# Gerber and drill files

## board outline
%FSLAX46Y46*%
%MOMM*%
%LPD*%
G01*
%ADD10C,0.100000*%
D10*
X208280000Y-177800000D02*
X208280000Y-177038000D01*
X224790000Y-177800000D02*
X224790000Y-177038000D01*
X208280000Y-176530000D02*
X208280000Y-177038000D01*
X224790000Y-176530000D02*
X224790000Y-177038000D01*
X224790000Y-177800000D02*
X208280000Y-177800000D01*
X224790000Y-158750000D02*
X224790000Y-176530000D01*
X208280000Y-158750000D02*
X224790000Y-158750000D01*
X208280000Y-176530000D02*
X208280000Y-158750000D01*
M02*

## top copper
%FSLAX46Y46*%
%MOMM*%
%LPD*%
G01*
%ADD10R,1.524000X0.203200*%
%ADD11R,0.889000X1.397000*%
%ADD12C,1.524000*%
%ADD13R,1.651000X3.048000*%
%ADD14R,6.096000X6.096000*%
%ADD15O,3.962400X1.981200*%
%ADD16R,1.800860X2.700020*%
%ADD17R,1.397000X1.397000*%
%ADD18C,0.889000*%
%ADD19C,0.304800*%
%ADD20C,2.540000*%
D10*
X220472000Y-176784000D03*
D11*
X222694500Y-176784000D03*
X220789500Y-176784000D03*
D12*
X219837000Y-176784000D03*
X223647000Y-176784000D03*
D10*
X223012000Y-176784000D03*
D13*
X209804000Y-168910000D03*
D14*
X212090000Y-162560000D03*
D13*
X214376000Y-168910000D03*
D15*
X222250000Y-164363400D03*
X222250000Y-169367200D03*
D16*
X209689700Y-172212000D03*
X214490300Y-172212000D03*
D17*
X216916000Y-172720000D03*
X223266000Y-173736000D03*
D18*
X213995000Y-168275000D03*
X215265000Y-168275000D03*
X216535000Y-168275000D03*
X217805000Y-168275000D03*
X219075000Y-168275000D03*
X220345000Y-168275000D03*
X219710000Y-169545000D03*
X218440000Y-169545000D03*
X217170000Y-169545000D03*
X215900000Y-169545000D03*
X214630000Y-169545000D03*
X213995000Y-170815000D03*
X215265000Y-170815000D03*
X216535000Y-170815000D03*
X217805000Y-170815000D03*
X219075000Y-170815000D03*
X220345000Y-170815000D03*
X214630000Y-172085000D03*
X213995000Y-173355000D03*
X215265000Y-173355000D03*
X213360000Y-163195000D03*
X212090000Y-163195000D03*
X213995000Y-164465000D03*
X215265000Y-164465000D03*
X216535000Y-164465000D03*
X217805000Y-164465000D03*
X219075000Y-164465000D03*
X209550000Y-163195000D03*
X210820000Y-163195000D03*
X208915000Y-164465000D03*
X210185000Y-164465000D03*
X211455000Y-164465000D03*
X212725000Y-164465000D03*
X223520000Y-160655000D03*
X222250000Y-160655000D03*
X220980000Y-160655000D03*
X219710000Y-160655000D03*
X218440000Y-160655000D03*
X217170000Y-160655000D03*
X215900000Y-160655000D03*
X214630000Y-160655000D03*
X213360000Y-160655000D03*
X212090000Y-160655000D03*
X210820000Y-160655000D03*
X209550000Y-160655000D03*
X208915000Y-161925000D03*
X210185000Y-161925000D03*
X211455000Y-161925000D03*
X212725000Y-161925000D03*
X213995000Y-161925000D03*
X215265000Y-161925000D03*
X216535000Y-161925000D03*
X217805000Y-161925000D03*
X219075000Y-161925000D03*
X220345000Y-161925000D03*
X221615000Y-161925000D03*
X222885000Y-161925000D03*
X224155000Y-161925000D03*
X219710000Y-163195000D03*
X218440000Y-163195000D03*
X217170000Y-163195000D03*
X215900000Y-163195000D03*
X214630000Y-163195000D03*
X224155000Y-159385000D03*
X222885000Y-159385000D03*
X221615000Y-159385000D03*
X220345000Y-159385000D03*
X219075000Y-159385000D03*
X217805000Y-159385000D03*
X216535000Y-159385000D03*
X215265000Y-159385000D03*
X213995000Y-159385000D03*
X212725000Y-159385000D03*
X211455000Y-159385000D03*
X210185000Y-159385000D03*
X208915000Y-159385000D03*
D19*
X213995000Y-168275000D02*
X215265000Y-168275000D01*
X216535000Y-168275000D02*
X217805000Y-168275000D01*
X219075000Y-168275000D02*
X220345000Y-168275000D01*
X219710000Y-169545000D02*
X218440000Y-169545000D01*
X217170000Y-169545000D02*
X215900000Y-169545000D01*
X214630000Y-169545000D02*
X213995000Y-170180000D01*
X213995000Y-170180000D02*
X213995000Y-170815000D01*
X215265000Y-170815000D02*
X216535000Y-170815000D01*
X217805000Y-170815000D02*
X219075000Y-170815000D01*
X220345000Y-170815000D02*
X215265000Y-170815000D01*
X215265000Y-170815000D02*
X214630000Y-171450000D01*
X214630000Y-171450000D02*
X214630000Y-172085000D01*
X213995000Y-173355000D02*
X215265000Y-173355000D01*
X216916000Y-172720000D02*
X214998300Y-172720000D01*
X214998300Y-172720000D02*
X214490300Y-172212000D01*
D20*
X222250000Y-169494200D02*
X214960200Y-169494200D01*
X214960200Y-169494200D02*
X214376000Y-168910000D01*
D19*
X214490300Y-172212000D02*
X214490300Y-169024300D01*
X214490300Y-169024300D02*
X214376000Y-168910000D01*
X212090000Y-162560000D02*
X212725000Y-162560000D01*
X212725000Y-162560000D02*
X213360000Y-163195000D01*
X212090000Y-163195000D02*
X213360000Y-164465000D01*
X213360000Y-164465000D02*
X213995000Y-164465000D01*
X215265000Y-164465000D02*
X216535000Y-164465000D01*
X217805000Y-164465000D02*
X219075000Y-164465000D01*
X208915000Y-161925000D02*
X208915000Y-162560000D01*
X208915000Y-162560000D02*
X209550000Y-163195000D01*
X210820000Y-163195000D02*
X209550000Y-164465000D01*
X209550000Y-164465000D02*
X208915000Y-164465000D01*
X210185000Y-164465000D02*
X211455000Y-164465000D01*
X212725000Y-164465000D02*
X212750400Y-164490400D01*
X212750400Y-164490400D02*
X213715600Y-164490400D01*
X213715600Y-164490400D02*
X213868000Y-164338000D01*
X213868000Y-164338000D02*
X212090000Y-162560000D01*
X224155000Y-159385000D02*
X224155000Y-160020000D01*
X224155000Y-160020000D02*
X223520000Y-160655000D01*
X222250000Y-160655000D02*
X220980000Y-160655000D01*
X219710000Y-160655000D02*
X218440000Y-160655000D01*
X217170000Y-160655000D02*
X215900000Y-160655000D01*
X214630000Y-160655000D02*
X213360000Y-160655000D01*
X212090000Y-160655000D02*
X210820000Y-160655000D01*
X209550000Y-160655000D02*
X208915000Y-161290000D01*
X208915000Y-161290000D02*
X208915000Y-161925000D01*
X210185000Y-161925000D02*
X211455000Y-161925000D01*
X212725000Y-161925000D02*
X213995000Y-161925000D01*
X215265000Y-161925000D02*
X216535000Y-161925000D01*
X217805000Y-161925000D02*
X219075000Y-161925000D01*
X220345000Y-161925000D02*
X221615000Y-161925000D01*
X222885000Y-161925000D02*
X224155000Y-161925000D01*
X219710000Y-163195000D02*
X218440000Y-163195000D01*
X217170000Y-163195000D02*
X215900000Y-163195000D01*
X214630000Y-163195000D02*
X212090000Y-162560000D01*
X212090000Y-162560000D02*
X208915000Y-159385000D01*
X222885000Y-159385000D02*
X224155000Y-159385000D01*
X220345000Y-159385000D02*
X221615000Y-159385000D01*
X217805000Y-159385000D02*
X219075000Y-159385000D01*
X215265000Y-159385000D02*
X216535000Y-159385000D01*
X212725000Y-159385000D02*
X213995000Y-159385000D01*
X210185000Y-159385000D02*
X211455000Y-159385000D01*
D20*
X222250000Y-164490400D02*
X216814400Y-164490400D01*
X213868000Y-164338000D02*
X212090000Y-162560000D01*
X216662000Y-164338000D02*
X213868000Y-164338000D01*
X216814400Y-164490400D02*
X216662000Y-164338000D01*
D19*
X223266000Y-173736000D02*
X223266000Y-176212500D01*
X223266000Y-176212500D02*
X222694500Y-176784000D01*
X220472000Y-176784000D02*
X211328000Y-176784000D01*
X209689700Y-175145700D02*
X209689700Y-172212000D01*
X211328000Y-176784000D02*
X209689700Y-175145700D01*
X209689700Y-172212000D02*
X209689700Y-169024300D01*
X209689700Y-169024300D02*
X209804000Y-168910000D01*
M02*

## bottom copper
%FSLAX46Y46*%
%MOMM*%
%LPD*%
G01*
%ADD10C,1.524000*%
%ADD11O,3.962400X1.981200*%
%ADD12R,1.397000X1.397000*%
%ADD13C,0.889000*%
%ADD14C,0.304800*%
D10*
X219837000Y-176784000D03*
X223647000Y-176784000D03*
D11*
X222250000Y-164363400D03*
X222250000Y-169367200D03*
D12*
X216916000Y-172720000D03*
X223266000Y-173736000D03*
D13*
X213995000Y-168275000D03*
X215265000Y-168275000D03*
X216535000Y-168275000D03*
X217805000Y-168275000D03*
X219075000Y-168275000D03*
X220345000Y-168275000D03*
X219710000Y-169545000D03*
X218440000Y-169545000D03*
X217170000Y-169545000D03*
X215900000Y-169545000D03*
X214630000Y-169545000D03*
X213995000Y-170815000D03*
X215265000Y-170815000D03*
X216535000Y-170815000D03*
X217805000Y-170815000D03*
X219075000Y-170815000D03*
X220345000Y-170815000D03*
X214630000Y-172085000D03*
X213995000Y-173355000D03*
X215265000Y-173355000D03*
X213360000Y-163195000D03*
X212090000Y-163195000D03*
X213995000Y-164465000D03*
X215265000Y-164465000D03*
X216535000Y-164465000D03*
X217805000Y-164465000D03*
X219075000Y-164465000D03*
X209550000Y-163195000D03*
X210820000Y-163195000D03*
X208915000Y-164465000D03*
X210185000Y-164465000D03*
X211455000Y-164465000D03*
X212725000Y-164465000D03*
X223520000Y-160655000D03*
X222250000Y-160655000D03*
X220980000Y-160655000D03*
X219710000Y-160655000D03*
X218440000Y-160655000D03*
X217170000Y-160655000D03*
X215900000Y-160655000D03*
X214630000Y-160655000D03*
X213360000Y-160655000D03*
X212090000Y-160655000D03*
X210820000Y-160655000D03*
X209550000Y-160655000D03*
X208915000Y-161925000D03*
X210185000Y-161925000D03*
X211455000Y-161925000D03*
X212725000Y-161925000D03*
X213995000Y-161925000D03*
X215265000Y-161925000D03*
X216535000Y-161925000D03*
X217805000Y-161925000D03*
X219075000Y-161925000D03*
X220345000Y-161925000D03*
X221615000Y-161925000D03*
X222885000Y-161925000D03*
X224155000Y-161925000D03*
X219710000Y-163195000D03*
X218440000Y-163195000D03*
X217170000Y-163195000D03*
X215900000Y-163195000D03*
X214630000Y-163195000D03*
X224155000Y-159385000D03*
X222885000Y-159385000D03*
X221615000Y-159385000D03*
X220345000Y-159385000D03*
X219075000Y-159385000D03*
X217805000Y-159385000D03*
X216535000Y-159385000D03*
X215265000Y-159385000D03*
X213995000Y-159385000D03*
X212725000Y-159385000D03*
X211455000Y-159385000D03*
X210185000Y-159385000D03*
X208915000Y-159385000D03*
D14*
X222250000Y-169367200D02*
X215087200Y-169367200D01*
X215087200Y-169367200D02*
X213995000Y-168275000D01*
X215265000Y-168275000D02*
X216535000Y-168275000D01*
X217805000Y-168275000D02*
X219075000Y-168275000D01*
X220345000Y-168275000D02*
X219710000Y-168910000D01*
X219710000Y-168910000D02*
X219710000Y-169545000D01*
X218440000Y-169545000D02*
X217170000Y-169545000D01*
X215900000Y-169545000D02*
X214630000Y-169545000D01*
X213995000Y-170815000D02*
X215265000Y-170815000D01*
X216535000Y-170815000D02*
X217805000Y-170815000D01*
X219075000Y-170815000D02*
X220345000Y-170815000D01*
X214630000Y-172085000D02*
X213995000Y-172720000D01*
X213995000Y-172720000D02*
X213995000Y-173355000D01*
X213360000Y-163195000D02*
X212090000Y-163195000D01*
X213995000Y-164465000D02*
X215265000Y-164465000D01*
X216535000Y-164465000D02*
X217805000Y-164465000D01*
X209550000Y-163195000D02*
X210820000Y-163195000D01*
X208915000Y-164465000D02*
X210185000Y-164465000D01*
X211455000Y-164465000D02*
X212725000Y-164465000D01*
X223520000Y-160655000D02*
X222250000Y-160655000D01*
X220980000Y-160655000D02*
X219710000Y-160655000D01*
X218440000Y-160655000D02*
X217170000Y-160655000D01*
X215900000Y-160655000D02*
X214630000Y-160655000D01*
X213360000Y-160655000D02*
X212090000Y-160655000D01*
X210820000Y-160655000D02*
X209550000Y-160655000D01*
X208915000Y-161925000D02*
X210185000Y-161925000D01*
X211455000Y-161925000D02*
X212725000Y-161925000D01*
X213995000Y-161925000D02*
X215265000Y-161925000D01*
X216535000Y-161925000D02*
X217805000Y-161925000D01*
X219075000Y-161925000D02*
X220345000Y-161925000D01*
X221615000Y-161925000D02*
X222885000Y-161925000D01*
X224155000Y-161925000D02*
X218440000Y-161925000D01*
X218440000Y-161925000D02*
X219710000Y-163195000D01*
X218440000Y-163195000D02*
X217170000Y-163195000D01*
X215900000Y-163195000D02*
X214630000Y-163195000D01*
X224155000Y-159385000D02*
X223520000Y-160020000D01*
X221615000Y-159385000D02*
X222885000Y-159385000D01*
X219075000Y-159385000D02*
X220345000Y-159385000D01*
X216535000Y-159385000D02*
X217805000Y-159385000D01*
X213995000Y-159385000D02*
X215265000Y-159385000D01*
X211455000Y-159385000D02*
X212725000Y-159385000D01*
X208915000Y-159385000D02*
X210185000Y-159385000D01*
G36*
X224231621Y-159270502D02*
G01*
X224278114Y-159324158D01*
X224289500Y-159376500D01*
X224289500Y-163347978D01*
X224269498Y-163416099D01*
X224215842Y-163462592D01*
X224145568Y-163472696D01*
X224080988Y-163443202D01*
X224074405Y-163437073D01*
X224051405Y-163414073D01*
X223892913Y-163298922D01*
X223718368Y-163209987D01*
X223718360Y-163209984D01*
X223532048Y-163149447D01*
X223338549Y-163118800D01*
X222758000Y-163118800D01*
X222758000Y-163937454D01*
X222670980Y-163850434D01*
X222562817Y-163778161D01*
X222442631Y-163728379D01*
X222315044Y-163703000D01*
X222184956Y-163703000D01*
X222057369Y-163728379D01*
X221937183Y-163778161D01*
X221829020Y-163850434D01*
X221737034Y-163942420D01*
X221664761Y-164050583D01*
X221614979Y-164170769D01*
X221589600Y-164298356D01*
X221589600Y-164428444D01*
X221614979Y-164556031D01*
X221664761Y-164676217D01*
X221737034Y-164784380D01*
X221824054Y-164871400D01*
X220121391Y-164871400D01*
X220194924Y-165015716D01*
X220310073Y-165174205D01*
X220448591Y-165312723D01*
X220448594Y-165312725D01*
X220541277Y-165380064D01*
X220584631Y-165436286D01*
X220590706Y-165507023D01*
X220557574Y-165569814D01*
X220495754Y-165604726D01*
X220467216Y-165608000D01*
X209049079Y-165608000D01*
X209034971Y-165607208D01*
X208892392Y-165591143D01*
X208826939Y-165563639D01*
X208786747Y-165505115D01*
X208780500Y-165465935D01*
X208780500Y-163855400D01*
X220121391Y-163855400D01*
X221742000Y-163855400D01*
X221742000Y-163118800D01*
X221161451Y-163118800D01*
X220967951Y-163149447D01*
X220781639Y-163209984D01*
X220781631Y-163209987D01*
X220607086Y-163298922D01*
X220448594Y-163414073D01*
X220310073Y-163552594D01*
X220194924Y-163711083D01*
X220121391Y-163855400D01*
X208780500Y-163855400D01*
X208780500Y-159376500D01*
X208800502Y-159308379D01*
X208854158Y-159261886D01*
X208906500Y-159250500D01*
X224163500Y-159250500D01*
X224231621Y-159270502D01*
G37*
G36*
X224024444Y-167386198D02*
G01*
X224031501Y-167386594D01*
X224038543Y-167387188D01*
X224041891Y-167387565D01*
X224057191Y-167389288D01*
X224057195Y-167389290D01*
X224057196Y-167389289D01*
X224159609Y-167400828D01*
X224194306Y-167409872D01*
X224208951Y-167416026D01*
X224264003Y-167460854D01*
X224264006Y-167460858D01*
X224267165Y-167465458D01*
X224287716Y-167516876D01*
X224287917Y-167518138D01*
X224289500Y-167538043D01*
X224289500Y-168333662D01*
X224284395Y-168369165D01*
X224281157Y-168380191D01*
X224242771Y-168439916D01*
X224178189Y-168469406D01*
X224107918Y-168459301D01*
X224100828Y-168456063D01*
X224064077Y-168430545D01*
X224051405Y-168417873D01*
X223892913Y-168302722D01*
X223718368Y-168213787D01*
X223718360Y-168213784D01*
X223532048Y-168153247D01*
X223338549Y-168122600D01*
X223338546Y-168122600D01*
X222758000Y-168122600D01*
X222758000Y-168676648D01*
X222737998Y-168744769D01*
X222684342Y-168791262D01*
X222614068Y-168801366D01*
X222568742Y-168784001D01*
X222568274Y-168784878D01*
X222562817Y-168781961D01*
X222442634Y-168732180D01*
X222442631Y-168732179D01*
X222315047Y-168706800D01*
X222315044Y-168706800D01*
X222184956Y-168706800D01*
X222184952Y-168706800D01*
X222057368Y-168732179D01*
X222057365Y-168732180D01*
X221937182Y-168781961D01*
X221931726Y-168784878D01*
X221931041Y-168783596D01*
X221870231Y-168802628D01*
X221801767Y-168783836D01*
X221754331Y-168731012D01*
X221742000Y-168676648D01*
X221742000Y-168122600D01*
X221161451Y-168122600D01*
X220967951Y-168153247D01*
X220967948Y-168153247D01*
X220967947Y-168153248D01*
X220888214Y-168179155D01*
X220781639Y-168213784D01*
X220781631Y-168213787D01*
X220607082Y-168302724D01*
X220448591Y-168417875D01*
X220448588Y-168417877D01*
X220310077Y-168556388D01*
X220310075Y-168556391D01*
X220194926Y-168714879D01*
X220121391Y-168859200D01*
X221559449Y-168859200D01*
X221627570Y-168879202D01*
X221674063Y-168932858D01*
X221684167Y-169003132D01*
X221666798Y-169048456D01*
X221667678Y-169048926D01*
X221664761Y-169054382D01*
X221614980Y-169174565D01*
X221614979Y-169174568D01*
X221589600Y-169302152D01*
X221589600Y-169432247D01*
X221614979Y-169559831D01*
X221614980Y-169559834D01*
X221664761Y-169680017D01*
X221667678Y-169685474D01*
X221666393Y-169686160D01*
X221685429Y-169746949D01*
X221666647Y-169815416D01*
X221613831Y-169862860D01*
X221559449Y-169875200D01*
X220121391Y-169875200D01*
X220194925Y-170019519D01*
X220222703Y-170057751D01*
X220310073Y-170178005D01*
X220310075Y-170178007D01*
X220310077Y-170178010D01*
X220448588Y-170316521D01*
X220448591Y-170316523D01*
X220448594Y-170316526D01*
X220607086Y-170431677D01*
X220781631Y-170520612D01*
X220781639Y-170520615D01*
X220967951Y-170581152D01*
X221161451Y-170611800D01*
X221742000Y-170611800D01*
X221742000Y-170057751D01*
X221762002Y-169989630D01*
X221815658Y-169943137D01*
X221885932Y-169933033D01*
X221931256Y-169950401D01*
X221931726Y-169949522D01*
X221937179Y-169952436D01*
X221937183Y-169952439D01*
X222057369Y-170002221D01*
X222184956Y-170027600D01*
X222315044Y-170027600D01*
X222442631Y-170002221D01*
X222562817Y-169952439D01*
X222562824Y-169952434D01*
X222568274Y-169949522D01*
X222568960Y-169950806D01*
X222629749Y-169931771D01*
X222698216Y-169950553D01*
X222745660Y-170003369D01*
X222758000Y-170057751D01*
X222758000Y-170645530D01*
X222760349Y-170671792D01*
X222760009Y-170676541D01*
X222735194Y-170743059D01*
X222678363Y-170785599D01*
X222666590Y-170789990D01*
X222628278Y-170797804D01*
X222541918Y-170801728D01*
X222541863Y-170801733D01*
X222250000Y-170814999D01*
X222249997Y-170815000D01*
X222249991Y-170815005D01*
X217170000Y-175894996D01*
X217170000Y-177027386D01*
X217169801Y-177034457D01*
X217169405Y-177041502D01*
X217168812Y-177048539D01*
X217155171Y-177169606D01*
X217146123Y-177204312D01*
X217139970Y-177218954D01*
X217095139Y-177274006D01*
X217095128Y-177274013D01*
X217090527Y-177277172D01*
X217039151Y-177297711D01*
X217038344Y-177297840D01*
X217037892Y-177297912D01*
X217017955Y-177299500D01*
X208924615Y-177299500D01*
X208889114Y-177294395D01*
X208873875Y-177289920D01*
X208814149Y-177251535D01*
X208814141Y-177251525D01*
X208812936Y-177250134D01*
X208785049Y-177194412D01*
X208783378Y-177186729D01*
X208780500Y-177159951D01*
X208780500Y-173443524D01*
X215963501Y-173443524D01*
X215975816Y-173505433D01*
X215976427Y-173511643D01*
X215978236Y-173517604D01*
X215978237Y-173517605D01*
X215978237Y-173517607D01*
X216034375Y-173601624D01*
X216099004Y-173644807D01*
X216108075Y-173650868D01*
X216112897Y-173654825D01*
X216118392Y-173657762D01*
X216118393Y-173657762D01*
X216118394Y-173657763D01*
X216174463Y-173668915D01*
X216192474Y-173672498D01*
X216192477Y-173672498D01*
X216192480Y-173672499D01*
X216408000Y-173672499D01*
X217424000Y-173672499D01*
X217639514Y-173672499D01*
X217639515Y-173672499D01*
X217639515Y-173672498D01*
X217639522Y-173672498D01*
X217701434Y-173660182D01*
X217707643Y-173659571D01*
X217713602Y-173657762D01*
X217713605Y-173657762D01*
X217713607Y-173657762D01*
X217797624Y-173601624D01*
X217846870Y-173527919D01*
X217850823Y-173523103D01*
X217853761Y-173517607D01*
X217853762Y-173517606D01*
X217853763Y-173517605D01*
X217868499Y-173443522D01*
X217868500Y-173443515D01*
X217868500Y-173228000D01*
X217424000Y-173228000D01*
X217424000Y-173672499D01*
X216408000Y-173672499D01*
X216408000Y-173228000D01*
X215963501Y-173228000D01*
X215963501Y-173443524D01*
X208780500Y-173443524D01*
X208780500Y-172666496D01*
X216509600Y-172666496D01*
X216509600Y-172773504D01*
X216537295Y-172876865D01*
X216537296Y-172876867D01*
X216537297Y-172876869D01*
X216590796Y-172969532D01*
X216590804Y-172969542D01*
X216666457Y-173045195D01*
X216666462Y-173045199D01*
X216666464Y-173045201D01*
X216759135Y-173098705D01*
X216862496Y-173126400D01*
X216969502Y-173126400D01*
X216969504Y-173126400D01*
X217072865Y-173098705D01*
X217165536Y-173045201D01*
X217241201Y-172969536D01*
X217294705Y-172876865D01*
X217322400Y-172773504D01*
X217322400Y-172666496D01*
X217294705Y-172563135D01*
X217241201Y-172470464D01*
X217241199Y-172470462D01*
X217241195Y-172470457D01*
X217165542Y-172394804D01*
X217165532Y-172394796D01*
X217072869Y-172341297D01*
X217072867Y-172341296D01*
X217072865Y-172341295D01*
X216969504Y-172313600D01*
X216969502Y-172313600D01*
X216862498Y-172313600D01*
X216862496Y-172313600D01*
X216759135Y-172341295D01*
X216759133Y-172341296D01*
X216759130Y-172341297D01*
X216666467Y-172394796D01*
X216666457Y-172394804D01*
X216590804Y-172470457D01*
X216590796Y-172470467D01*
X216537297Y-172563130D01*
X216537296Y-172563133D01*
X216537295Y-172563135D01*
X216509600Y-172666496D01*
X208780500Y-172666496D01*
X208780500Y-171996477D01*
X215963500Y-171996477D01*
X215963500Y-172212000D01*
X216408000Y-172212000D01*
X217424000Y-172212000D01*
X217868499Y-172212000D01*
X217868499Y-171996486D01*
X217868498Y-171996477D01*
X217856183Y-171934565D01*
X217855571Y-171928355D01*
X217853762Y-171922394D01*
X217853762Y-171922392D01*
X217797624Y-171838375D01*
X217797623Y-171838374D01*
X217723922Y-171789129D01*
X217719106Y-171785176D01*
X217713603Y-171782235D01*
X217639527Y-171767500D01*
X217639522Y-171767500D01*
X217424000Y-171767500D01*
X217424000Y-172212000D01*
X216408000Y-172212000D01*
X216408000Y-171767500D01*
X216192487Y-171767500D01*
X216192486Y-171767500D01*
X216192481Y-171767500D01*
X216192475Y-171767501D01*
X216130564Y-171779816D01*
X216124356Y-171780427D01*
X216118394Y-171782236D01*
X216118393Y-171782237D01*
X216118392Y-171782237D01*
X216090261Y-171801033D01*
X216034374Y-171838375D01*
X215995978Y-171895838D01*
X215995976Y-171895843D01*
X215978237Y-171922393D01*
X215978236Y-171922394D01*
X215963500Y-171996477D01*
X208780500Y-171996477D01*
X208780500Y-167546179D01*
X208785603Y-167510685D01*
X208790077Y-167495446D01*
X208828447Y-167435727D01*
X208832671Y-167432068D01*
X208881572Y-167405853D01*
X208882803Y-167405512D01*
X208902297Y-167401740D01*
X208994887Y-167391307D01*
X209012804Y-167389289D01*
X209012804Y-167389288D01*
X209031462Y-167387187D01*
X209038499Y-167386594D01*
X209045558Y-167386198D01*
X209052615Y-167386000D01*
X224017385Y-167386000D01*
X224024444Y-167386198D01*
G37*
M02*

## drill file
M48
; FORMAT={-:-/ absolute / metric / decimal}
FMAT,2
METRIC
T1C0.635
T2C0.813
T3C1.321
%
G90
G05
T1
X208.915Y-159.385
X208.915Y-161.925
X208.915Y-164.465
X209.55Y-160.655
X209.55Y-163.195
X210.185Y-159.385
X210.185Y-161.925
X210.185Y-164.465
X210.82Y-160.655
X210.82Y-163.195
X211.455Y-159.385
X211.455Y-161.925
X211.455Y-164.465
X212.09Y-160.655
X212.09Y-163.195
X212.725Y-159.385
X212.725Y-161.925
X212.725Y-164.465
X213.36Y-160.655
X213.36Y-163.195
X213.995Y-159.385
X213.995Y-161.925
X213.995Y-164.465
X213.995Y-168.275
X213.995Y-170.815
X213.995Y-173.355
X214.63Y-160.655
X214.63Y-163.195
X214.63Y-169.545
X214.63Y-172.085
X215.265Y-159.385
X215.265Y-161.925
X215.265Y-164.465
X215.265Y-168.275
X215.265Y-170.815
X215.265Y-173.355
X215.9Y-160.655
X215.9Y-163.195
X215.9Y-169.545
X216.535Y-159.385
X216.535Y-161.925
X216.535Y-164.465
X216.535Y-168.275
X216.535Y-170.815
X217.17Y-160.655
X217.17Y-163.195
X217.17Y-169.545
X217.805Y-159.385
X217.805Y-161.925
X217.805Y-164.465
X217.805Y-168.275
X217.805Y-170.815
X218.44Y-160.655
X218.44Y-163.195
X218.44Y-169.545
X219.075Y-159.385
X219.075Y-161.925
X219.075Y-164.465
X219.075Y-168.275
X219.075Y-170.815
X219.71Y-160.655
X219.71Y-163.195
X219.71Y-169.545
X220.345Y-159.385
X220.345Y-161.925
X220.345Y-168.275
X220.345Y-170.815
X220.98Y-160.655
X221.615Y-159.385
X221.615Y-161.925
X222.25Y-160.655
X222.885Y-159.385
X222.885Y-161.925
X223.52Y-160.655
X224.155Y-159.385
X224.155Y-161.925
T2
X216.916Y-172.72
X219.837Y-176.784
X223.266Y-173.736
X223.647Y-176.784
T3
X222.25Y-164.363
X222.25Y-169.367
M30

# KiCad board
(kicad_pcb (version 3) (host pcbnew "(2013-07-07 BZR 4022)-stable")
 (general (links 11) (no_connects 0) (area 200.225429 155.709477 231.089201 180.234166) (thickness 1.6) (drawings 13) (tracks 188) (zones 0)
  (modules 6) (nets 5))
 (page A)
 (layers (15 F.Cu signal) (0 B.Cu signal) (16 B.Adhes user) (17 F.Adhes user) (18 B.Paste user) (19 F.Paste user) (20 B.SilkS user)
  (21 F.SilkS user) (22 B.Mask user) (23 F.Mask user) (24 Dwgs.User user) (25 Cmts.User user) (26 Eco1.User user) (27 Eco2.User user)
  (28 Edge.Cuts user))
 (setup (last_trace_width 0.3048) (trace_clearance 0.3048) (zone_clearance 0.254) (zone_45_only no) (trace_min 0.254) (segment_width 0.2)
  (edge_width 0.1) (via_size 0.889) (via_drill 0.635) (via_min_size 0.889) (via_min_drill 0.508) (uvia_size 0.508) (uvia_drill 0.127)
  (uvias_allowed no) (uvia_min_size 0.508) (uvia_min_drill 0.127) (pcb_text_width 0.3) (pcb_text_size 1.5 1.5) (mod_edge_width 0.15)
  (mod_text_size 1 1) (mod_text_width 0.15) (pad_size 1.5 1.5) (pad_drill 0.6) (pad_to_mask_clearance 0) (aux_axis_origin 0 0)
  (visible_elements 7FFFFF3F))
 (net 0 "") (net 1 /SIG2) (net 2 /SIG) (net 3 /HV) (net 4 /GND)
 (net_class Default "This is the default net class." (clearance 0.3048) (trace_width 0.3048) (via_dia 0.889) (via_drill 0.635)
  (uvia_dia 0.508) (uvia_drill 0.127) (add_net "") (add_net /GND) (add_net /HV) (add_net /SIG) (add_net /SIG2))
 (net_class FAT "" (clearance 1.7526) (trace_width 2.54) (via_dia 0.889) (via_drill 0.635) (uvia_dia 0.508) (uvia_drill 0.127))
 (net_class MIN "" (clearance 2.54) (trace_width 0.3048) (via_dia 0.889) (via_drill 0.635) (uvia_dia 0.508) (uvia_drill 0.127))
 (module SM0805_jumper (layer F.Cu) (at 221.742 176.784 180)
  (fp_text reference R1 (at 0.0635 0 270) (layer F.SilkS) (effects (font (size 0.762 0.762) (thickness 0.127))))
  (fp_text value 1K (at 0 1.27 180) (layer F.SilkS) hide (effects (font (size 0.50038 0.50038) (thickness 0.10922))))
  (pad 2 smd rect (at 1.27 0 180) (size 1.524 0.2032) (layers F.Cu F.Paste F.Mask) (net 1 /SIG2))
  (pad 1 smd rect (at -0.9525 0 180) (size 0.889 1.397) (layers F.Cu F.Paste F.Mask) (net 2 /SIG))
  (pad 2 smd rect (at 0.9525 0 180) (size 0.889 1.397) (layers F.Cu F.Paste F.Mask) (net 1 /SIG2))
  (pad 2 thru_hole circle (at 1.905 0 180) (size 1.524 1.524) (drill 0.8128) (layers *.Cu *.Mask F.SilkS) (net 1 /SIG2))
  (pad 1 thru_hole circle (at -1.905 0 180) (size 1.524 1.524) (drill 0.8128) (layers *.Cu *.Mask F.SilkS) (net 2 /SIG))
  (pad 1 smd rect (at -1.27 0 180) (size 1.524 0.2032) (layers F.Cu F.Paste F.Mask) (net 2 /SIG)))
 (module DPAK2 (layer F.Cu) (at 212.09 168.91)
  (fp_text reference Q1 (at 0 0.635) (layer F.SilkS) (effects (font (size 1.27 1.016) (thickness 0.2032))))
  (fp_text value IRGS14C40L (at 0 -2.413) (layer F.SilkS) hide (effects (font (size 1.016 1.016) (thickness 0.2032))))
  (pad 1 smd rect (at -2.286 0) (size 1.651 3.048) (layers F.Cu F.Paste F.Mask) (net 1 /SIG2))
  (pad 2 smd rect (at 0 -6.35) (size 6.096 6.096) (layers F.Cu F.Paste F.Mask) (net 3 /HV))
  (pad 3 smd rect (at 2.286 0) (size 1.651 3.048) (layers F.Cu F.Paste F.Mask) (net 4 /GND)))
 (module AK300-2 (layer F.Cu) (at 222.25 166.878 270)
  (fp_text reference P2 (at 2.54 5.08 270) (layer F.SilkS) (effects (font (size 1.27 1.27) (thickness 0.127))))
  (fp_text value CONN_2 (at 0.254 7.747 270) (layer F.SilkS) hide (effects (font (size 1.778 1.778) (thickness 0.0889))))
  (pad 1 thru_hole oval (at -2.5146 0 270) (size 1.9812 3.9624) (drill 1.3208) (layers *.Cu F.Paste F.SilkS F.Mask) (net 3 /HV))
  (pad 2 thru_hole oval (at 2.4892 0 270) (size 1.9812 3.9624) (drill 1.3208) (layers *.Cu F.Paste F.SilkS F.Mask) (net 4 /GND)))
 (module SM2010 (layer F.Cu) (at 212.09 172.212)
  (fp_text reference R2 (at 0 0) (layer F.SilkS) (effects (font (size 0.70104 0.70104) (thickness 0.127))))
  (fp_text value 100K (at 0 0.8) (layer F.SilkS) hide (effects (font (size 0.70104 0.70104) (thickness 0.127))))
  (pad 1 smd rect (at -2.4003 0) (size 1.80086 2.70002) (layers F.Cu F.Paste F.Mask) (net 1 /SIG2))
  (pad 2 smd rect (at 2.4003 0) (size 1.80086 2.70002) (layers F.Cu F.Paste F.Mask) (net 4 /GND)))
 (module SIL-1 (layer F.Cu) (at 216.916 172.72)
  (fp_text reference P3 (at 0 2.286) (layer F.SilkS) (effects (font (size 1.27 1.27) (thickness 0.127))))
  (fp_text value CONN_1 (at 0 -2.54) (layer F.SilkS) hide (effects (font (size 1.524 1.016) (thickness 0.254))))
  (pad 1 thru_hole rect (at 0 0) (size 1.397 1.397) (drill 0.8128) (layers *.Cu *.Mask F.SilkS) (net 4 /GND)))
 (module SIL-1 (layer F.Cu) (at 223.266 173.736 180)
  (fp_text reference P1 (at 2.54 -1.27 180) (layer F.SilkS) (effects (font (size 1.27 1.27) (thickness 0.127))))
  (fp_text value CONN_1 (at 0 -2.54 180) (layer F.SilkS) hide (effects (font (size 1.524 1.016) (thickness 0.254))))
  (pad 1 thru_hole rect (at 0 0 180) (size 1.397 1.397) (drill 0.8128) (layers *.Cu *.Mask F.SilkS) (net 2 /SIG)))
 (gr_line (start 208.28 177.8) (end 208.28 177.038) (angle 90) (layer Edge.Cuts) (width 0.1))
 (gr_line (start 224.79 177.8) (end 224.79 177.038) (angle 90) (layer Edge.Cuts) (width 0.1))
 (gr_line (start 208.28 176.53) (end 208.28 177.038) (angle 90) (layer Edge.Cuts) (width 0.1))
 (gr_line (start 224.79 176.53) (end 224.79 177.038) (angle 90) (layer Edge.Cuts) (width 0.1))
 (gr_line (start 224.79 177.8) (end 208.28 177.8) (angle 90) (layer Edge.Cuts) (width 0.1))
 (gr_line (start 224.79 158.75) (end 224.79 176.53) (angle 90) (layer Edge.Cuts) (width 0.1))
 (gr_line (start 208.28 158.75) (end 224.79 158.75) (angle 90) (layer Edge.Cuts) (width 0.1))
 (gr_line (start 208.28 176.53) (end 208.28 158.75) (angle 90) (layer Edge.Cuts) (width 0.1))
 (segment (start 222.25 169.3672) (end 215.0872 169.3672) (width 0.3048) (layer B.Cu) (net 4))
 (segment (start 215.0872 169.3672) (end 213.995 168.275) (width 0.3048) (layer B.Cu) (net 4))
 (via (at 213.995 168.275) (size 0.889) (layers F.Cu B.Cu) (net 4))
 (segment (start 213.995 168.275) (end 215.265 168.275) (width 0.3048) (layer F.Cu) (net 4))
 (via (at 215.265 168.275) (size 0.889) (layers F.Cu B.Cu) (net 4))
 (segment (start 215.265 168.275) (end 216.535 168.275) (width 0.3048) (layer B.Cu) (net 4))
 (via (at 216.535 168.275) (size 0.889) (layers F.Cu B.Cu) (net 4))
 (segment (start 216.535 168.275) (end 217.805 168.275) (width 0.3048) (layer F.Cu) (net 4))
 (via (at 217.805 168.275) (size 0.889) (layers F.Cu B.Cu) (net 4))
 (segment (start 217.805 168.275) (end 219.075 168.275) (width 0.3048) (layer B.Cu) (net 4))
 (via (at 219.075 168.275) (size 0.889) (layers F.Cu B.Cu) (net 4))
 (segment (start 219.075 168.275) (end 220.345 168.275) (width 0.3048) (layer F.Cu) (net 4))
 (via (at 220.345 168.275) (size 0.889) (layers F.Cu B.Cu) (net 4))
 (segment (start 220.345 168.275) (end 219.71 168.91) (width 0.3048) (layer B.Cu) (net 4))
 (segment (start 219.71 168.91) (end 219.71 169.545) (width 0.3048) (layer B.Cu) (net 4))
 (via (at 219.71 169.545) (size 0.889) (layers F.Cu B.Cu) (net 4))
 (segment (start 219.71 169.545) (end 218.44 169.545) (width 0.3048) (layer F.Cu) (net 4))
 (via (at 218.44 169.545) (size 0.889) (layers F.Cu B.Cu) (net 4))
 (segment (start 218.44 169.545) (end 217.17 169.545) (width 0.3048) (layer B.Cu) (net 4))
 (via (at 217.17 169.545) (size 0.889) (layers F.Cu B.Cu) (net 4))
 (segment (start 217.17 169.545) (end 215.9 169.545) (width 0.3048) (layer F.Cu) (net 4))
 (via (at 215.9 169.545) (size 0.889) (layers F.Cu B.Cu) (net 4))
 (segment (start 215.9 169.545) (end 214.63 169.545) (width 0.3048) (layer B.Cu) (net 4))
 (via (at 214.63 169.545) (size 0.889) (layers F.Cu B.Cu) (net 4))
 (segment (start 214.63 169.545) (end 213.995 170.18) (width 0.3048) (layer F.Cu) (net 4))
 (segment (start 213.995 170.18) (end 213.995 170.815) (width 0.3048) (layer F.Cu) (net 4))
 (via (at 213.995 170.815) (size 0.889) (layers F.Cu B.Cu) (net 4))
 (segment (start 213.995 170.815) (end 215.265 170.815) (width 0.3048) (layer B.Cu) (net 4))
 (via (at 215.265 170.815) (size 0.889) (layers F.Cu B.Cu) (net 4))
 (segment (start 215.265 170.815) (end 216.535 170.815) (width 0.3048) (layer F.Cu) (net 4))
 (via (at 216.535 170.815) (size 0.889) (layers F.Cu B.Cu) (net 4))
 (segment (start 216.535 170.815) (end 217.805 170.815) (width 0.3048) (layer B.Cu) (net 4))
 (via (at 217.805 170.815) (size 0.889) (layers F.Cu B.Cu) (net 4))
 (segment (start 217.805 170.815) (end 219.075 170.815) (width 0.3048) (layer F.Cu) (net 4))
 (via (at 219.075 170.815) (size 0.889) (layers F.Cu B.Cu) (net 4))
 (segment (start 219.075 170.815) (end 220.345 170.815) (width 0.3048) (layer B.Cu) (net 4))
 (via (at 220.345 170.815) (size 0.889) (layers F.Cu B.Cu) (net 4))
 (segment (start 220.345 170.815) (end 215.265 170.815) (width 0.3048) (layer F.Cu) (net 4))
 (segment (start 215.265 170.815) (end 214.63 171.45) (width 0.3048) (layer F.Cu) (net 4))
 (segment (start 214.63 171.45) (end 214.63 172.085) (width 0.3048) (layer F.Cu) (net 4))
 (via (at 214.63 172.085) (size 0.889) (layers F.Cu B.Cu) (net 4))
 (segment (start 214.63 172.085) (end 213.995 172.72) (width 0.3048) (layer B.Cu) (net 4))
 (segment (start 213.995 172.72) (end 213.995 173.355) (width 0.3048) (layer B.Cu) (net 4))
 (via (at 213.995 173.355) (size 0.889) (layers F.Cu B.Cu) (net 4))
 (segment (start 213.995 173.355) (end 215.265 173.355) (width 0.3048) (layer F.Cu) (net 4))
 (via (at 215.265 173.355) (size 0.889) (layers F.Cu B.Cu) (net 4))
 (segment (start 216.916 172.72) (end 214.9983 172.72) (width 0.3048) (layer F.Cu) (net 4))
 (segment (start 214.9983 172.72) (end 214.4903 172.212) (width 0.3048) (layer F.Cu) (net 4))
 (segment (start 222.25 169.4942) (end 214.9602 169.4942) (width 2.54) (layer F.Cu) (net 4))
 (segment (start 214.9602 169.4942) (end 214.376 168.91) (width 2.54) (layer F.Cu) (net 4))
 (segment (start 214.4903 172.212) (end 214.4903 169.0243) (width 0.3048) (layer F.Cu) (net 4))
 (segment (start 214.4903 169.0243) (end 214.376 168.91) (width 0.3048) (layer F.Cu) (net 4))
 (segment (start 212.09 162.56) (end 212.725 162.56) (width 0.3048) (layer F.Cu) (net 3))
 (segment (start 212.725 162.56) (end 213.36 163.195) (width 0.3048) (layer F.Cu) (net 3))
 (via (at 213.36 163.195) (size 0.889) (layers F.Cu B.Cu) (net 3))
 (segment (start 213.36 163.195) (end 212.09 163.195) (width 0.3048) (layer B.Cu) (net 3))
 (via (at 212.09 163.195) (size 0.889) (layers F.Cu B.Cu) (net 3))
 (segment (start 212.09 163.195) (end 213.36 164.465) (width 0.3048) (layer F.Cu) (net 3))
 (segment (start 213.36 164.465) (end 213.995 164.465) (width 0.3048) (layer F.Cu) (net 3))
 (via (at 213.995 164.465) (size 0.889) (layers F.Cu B.Cu) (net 3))
 (segment (start 213.995 164.465) (end 215.265 164.465) (width 0.3048) (layer B.Cu) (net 3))
 (via (at 215.265 164.465) (size 0.889) (layers F.Cu B.Cu) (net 3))
 (segment (start 215.265 164.465) (end 216.535 164.465) (width 0.3048) (layer F.Cu) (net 3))
 (via (at 216.535 164.465) (size 0.889) (layers F.Cu B.Cu) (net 3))
 (segment (start 216.535 164.465) (end 217.805 164.465) (width 0.3048) (layer B.Cu) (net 3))
 (via (at 217.805 164.465) (size 0.889) (layers F.Cu B.Cu) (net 3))
 (segment (start 217.805 164.465) (end 219.075 164.465) (width 0.3048) (layer F.Cu) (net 3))
 (via (at 219.075 164.465) (size 0.889) (layers F.Cu B.Cu) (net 3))
 (segment (start 208.915 161.925) (end 208.915 162.56) (width 0.3048) (layer F.Cu) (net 3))
 (segment (start 208.915 162.56) (end 209.55 163.195) (width 0.3048) (layer F.Cu) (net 3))
 (via (at 209.55 163.195) (size 0.889) (layers F.Cu B.Cu) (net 3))
 (segment (start 209.55 163.195) (end 210.82 163.195) (width 0.3048) (layer B.Cu) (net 3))
 (via (at 210.82 163.195) (size 0.889) (layers F.Cu B.Cu) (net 3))
 (segment (start 210.82 163.195) (end 209.55 164.465) (width 0.3048) (layer F.Cu) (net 3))
 (segment (start 209.55 164.465) (end 208.915 164.465) (width 0.3048) (layer F.Cu) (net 3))
 (via (at 208.915 164.465) (size 0.889) (layers F.Cu B.Cu) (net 3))
 (segment (start 208.915 164.465) (end 210.185 164.465) (width 0.3048) (layer B.Cu) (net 3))
 (via (at 210.185 164.465) (size 0.889) (layers F.Cu B.Cu) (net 3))
 (segment (start 210.185 164.465) (end 211.455 164.465) (width 0.3048) (layer F.Cu) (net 3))
 (via (at 211.455 164.465) (size 0.889) (layers F.Cu B.Cu) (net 3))
 (segment (start 211.455 164.465) (end 212.725 164.465) (width 0.3048) (layer B.Cu) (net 3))
 (via (at 212.725 164.465) (size 0.889) (layers F.Cu B.Cu) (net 3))
 (segment (start 212.725 164.465) (end 212.7504 164.4904) (width 0.3048) (layer F.Cu) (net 3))
 (segment (start 212.7504 164.4904) (end 213.7156 164.4904) (width 0.3048) (layer F.Cu) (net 3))
 (segment (start 213.7156 164.4904) (end 213.868 164.338) (width 0.3048) (layer F.Cu) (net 3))
 (segment (start 213.868 164.338) (end 212.09 162.56) (width 0.3048) (layer F.Cu) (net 3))
 (segment (start 224.155 159.385) (end 224.155 160.02) (width 0.3048) (layer F.Cu) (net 3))
 (segment (start 224.155 160.02) (end 223.52 160.655) (width 0.3048) (layer F.Cu) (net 3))
 (via (at 223.52 160.655) (size 0.889) (layers F.Cu B.Cu) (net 3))
 (segment (start 223.52 160.655) (end 222.25 160.655) (width 0.3048) (layer B.Cu) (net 3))
 (via (at 222.25 160.655) (size 0.889) (layers F.Cu B.Cu) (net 3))
 (segment (start 222.25 160.655) (end 220.98 160.655) (width 0.3048) (layer F.Cu) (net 3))
 (via (at 220.98 160.655) (size 0.889) (layers F.Cu B.Cu) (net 3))
 (segment (start 220.98 160.655) (end 219.71 160.655) (width 0.3048) (layer B.Cu) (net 3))
 (via (at 219.71 160.655) (size 0.889) (layers F.Cu B.Cu) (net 3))
 (segment (start 219.71 160.655) (end 218.44 160.655) (width 0.3048) (layer F.Cu) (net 3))
 (via (at 218.44 160.655) (size 0.889) (layers F.Cu B.Cu) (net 3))
 (segment (start 218.44 160.655) (end 217.17 160.655) (width 0.3048) (layer B.Cu) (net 3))
 (via (at 217.17 160.655) (size 0.889) (layers F.Cu B.Cu) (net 3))
 (segment (start 217.17 160.655) (end 215.9 160.655) (width 0.3048) (layer F.Cu) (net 3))
 (via (at 215.9 160.655) (size 0.889) (layers F.Cu B.Cu) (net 3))
 (segment (start 215.9 160.655) (end 214.63 160.655) (width 0.3048) (layer B.Cu) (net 3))
 (via (at 214.63 160.655) (size 0.889) (layers F.Cu B.Cu) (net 3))
 (segment (start 214.63 160.655) (end 213.36 160.655) (width 0.3048) (layer F.Cu) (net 3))
 (via (at 213.36 160.655) (size 0.889) (layers F.Cu B.Cu) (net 3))
 (segment (start 213.36 160.655) (end 212.09 160.655) (width 0.3048) (layer B.Cu) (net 3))
 (via (at 212.09 160.655) (size 0.889) (layers F.Cu B.Cu) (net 3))
 (segment (start 212.09 160.655) (end 210.82 160.655) (width 0.3048) (layer F.Cu) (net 3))
 (via (at 210.82 160.655) (size 0.889) (layers F.Cu B.Cu) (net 3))
 (segment (start 210.82 160.655) (end 209.55 160.655) (width 0.3048) (layer B.Cu) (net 3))
 (via (at 209.55 160.655) (size 0.889) (layers F.Cu B.Cu) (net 3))
 (segment (start 209.55 160.655) (end 208.915 161.29) (width 0.3048) (layer F.Cu) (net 3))
 (segment (start 208.915 161.29) (end 208.915 161.925) (width 0.3048) (layer F.Cu) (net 3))
 (via (at 208.915 161.925) (size 0.889) (layers F.Cu B.Cu) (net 3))
 (segment (start 208.915 161.925) (end 210.185 161.925) (width 0.3048) (layer B.Cu) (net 3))
 (via (at 210.185 161.925) (size 0.889) (layers F.Cu B.Cu) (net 3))
 (segment (start 210.185 161.925) (end 211.455 161.925) (width 0.3048) (layer F.Cu) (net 3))
 (via (at 211.455 161.925) (size 0.889) (layers F.Cu B.Cu) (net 3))
 (segment (start 211.455 161.925) (end 212.725 161.925) (width 0.3048) (layer B.Cu) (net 3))
 (via (at 212.725 161.925) (size 0.889) (layers F.Cu B.Cu) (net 3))
 (segment (start 212.725 161.925) (end 213.995 161.925) (width 0.3048) (layer F.Cu) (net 3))
 (via (at 213.995 161.925) (size 0.889) (layers F.Cu B.Cu) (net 3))
 (segment (start 213.995 161.925) (end 215.265 161.925) (width 0.3048) (layer B.Cu) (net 3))
 (via (at 215.265 161.925) (size 0.889) (layers F.Cu B.Cu) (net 3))
 (segment (start 215.265 161.925) (end 216.535 161.925) (width 0.3048) (layer F.Cu) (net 3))
 (via (at 216.535 161.925) (size 0.889) (layers F.Cu B.Cu) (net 3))
 (segment (start 216.535 161.925) (end 217.805 161.925) (width 0.3048) (layer B.Cu) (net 3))
 (via (at 217.805 161.925) (size 0.889) (layers F.Cu B.Cu) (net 3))
 (segment (start 217.805 161.925) (end 219.075 161.925) (width 0.3048) (layer F.Cu) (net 3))
 (via (at 219.075 161.925) (size 0.889) (layers F.Cu B.Cu) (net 3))
 (segment (start 219.075 161.925) (end 220.345 161.925) (width 0.3048) (layer B.Cu) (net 3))
 (via (at 220.345 161.925) (size 0.889) (layers F.Cu B.Cu) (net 3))
 (segment (start 220.345 161.925) (end 221.615 161.925) (width 0.3048) (layer F.Cu) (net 3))
 (via (at 221.615 161.925) (size 0.889) (layers F.Cu B.Cu) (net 3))
 (segment (start 221.615 161.925) (end 222.885 161.925) (width 0.3048) (layer B.Cu) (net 3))
 (via (at 222.885 161.925) (size 0.889) (layers F.Cu B.Cu) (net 3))
 (segment (start 222.885 161.925) (end 224.155 161.925) (width 0.3048) (layer F.Cu) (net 3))
 (via (at 224.155 161.925) (size 0.889) (layers F.Cu B.Cu) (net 3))
 (segment (start 224.155 161.925) (end 218.44 161.925) (width 0.3048) (layer B.Cu) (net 3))
 (segment (start 218.44 161.925) (end 219.71 163.195) (width 0.3048) (layer B.Cu) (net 3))
 (via (at 219.71 163.195) (size 0.889) (layers F.Cu B.Cu) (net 3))
 (segment (start 219.71 163.195) (end 218.44 163.195) (width 0.3048) (layer F.Cu) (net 3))
 (via (at 218.44 163.195) (size 0.889) (layers F.Cu B.Cu) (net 3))
 (segment (start 218.44 163.195) (end 217.17 163.195) (width 0.3048) (layer B.Cu) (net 3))
 (via (at 217.17 163.195) (size 0.889) (layers F.Cu B.Cu) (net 3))
 (segment (start 217.17 163.195) (end 215.9 163.195) (width 0.3048) (layer F.Cu) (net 3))
 (via (at 215.9 163.195) (size 0.889) (layers F.Cu B.Cu) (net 3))
 (segment (start 215.9 163.195) (end 214.63 163.195) (width 0.3048) (layer B.Cu) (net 3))
 (via (at 214.63 163.195) (size 0.889) (layers F.Cu B.Cu) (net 3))
 (segment (start 214.63 163.195) (end 212.09 162.56) (width 0.3048) (layer F.Cu) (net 3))
 (segment (start 212.09 162.56) (end 208.915 159.385) (width 0.3048) (layer F.Cu) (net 3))
 (segment (start 224.155 159.385) (end 223.52 160.02) (width 0.3048) (layer B.Cu) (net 3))
 (via (at 224.155 159.385) (size 0.889) (layers F.Cu B.Cu) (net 3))
 (segment (start 222.885 159.385) (end 224.155 159.385) (width 0.3048) (layer F.Cu) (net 3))
 (via (at 222.885 159.385) (size 0.889) (layers F.Cu B.Cu) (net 3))
 (segment (start 221.615 159.385) (end 222.885 159.385) (width 0.3048) (layer B.Cu) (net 3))
 (via (at 221.615 159.385) (size 0.889) (layers F.Cu B.Cu) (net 3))
 (segment (start 220.345 159.385) (end 221.615 159.385) (width 0.3048) (layer F.Cu) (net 3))
 (via (at 220.345 159.385) (size 0.889) (layers F.Cu B.Cu) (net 3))
 (segment (start 219.075 159.385) (end 220.345 159.385) (width 0.3048) (layer B.Cu) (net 3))
 (via (at 219.075 159.385) (size 0.889) (layers F.Cu B.Cu) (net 3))
 (segment (start 217.805 159.385) (end 219.075 159.385) (width 0.3048) (layer F.Cu) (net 3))
 (via (at 217.805 159.385) (size 0.889) (layers F.Cu B.Cu) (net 3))
 (segment (start 216.535 159.385) (end 217.805 159.385) (width 0.3048) (layer B.Cu) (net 3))
 (via (at 216.535 159.385) (size 0.889) (layers F.Cu B.Cu) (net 3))
 (segment (start 215.265 159.385) (end 216.535 159.385) (width 0.3048) (layer F.Cu) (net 3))
 (via (at 215.265 159.385) (size 0.889) (layers F.Cu B.Cu) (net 3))
 (segment (start 213.995 159.385) (end 215.265 159.385) (width 0.3048) (layer B.Cu) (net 3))
 (via (at 213.995 159.385) (size 0.889) (layers F.Cu B.Cu) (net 3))
 (segment (start 212.725 159.385) (end 213.995 159.385) (width 0.3048) (layer F.Cu) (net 3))
 (via (at 212.725 159.385) (size 0.889) (layers F.Cu B.Cu) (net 3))
 (segment (start 211.455 159.385) (end 212.725 159.385) (width 0.3048) (layer B.Cu) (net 3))
 (via (at 211.455 159.385) (size 0.889) (layers F.Cu B.Cu) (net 3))
 (segment (start 210.185 159.385) (end 211.455 159.385) (width 0.3048) (layer F.Cu) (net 3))
 (via (at 210.185 159.385) (size 0.889) (layers F.Cu B.Cu) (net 3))
 (segment (start 208.915 159.385) (end 210.185 159.385) (width 0.3048) (layer B.Cu) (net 3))
 (via (at 208.915 159.385) (size 0.889) (layers F.Cu B.Cu) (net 3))
 (segment (start 222.25 164.4904) (end 216.8144 164.4904) (width 2.54) (layer F.Cu) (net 3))
 (segment (start 213.868 164.338) (end 212.09 162.56) (width 2.54) (layer F.Cu) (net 3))
 (segment (start 216.662 164.338) (end 213.868 164.338) (width 2.54) (layer F.Cu) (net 3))
 (segment (start 216.8144 164.4904) (end 216.662 164.338) (width 2.54) (layer F.Cu) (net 3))
 (segment (start 223.266 173.736) (end 223.266 176.2125) (width 0.3048) (layer F.Cu) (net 2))
 (segment (start 223.266 176.2125) (end 222.6945 176.784) (width 0.3048) (layer F.Cu) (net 2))
 (segment (start 220.472 176.784) (end 211.328 176.784) (width 0.3048) (layer F.Cu) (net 1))
 (segment (start 209.6897 175.1457) (end 209.6897 172.212) (width 0.3048) (layer F.Cu) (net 1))
 (segment (start 211.328 176.784) (end 209.6897 175.1457) (width 0.3048) (layer F.Cu) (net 1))
 (segment (start 209.6897 172.212) (end 209.6897 169.0243) (width 0.3048) (layer F.Cu) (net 1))
 (segment (start 209.6897 169.0243) (end 209.804 168.91) (width 0.3048) (layer F.Cu) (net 1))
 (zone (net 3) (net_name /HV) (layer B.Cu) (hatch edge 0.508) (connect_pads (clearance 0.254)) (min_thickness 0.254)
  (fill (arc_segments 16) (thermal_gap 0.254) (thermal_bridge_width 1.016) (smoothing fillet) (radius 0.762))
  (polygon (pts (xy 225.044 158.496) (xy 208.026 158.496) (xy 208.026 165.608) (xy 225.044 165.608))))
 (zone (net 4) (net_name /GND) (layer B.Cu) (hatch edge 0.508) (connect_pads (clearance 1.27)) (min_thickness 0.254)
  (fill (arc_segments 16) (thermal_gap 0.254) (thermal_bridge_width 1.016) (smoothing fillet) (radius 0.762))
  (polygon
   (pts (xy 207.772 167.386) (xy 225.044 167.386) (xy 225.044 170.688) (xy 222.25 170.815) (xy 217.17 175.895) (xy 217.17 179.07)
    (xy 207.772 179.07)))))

